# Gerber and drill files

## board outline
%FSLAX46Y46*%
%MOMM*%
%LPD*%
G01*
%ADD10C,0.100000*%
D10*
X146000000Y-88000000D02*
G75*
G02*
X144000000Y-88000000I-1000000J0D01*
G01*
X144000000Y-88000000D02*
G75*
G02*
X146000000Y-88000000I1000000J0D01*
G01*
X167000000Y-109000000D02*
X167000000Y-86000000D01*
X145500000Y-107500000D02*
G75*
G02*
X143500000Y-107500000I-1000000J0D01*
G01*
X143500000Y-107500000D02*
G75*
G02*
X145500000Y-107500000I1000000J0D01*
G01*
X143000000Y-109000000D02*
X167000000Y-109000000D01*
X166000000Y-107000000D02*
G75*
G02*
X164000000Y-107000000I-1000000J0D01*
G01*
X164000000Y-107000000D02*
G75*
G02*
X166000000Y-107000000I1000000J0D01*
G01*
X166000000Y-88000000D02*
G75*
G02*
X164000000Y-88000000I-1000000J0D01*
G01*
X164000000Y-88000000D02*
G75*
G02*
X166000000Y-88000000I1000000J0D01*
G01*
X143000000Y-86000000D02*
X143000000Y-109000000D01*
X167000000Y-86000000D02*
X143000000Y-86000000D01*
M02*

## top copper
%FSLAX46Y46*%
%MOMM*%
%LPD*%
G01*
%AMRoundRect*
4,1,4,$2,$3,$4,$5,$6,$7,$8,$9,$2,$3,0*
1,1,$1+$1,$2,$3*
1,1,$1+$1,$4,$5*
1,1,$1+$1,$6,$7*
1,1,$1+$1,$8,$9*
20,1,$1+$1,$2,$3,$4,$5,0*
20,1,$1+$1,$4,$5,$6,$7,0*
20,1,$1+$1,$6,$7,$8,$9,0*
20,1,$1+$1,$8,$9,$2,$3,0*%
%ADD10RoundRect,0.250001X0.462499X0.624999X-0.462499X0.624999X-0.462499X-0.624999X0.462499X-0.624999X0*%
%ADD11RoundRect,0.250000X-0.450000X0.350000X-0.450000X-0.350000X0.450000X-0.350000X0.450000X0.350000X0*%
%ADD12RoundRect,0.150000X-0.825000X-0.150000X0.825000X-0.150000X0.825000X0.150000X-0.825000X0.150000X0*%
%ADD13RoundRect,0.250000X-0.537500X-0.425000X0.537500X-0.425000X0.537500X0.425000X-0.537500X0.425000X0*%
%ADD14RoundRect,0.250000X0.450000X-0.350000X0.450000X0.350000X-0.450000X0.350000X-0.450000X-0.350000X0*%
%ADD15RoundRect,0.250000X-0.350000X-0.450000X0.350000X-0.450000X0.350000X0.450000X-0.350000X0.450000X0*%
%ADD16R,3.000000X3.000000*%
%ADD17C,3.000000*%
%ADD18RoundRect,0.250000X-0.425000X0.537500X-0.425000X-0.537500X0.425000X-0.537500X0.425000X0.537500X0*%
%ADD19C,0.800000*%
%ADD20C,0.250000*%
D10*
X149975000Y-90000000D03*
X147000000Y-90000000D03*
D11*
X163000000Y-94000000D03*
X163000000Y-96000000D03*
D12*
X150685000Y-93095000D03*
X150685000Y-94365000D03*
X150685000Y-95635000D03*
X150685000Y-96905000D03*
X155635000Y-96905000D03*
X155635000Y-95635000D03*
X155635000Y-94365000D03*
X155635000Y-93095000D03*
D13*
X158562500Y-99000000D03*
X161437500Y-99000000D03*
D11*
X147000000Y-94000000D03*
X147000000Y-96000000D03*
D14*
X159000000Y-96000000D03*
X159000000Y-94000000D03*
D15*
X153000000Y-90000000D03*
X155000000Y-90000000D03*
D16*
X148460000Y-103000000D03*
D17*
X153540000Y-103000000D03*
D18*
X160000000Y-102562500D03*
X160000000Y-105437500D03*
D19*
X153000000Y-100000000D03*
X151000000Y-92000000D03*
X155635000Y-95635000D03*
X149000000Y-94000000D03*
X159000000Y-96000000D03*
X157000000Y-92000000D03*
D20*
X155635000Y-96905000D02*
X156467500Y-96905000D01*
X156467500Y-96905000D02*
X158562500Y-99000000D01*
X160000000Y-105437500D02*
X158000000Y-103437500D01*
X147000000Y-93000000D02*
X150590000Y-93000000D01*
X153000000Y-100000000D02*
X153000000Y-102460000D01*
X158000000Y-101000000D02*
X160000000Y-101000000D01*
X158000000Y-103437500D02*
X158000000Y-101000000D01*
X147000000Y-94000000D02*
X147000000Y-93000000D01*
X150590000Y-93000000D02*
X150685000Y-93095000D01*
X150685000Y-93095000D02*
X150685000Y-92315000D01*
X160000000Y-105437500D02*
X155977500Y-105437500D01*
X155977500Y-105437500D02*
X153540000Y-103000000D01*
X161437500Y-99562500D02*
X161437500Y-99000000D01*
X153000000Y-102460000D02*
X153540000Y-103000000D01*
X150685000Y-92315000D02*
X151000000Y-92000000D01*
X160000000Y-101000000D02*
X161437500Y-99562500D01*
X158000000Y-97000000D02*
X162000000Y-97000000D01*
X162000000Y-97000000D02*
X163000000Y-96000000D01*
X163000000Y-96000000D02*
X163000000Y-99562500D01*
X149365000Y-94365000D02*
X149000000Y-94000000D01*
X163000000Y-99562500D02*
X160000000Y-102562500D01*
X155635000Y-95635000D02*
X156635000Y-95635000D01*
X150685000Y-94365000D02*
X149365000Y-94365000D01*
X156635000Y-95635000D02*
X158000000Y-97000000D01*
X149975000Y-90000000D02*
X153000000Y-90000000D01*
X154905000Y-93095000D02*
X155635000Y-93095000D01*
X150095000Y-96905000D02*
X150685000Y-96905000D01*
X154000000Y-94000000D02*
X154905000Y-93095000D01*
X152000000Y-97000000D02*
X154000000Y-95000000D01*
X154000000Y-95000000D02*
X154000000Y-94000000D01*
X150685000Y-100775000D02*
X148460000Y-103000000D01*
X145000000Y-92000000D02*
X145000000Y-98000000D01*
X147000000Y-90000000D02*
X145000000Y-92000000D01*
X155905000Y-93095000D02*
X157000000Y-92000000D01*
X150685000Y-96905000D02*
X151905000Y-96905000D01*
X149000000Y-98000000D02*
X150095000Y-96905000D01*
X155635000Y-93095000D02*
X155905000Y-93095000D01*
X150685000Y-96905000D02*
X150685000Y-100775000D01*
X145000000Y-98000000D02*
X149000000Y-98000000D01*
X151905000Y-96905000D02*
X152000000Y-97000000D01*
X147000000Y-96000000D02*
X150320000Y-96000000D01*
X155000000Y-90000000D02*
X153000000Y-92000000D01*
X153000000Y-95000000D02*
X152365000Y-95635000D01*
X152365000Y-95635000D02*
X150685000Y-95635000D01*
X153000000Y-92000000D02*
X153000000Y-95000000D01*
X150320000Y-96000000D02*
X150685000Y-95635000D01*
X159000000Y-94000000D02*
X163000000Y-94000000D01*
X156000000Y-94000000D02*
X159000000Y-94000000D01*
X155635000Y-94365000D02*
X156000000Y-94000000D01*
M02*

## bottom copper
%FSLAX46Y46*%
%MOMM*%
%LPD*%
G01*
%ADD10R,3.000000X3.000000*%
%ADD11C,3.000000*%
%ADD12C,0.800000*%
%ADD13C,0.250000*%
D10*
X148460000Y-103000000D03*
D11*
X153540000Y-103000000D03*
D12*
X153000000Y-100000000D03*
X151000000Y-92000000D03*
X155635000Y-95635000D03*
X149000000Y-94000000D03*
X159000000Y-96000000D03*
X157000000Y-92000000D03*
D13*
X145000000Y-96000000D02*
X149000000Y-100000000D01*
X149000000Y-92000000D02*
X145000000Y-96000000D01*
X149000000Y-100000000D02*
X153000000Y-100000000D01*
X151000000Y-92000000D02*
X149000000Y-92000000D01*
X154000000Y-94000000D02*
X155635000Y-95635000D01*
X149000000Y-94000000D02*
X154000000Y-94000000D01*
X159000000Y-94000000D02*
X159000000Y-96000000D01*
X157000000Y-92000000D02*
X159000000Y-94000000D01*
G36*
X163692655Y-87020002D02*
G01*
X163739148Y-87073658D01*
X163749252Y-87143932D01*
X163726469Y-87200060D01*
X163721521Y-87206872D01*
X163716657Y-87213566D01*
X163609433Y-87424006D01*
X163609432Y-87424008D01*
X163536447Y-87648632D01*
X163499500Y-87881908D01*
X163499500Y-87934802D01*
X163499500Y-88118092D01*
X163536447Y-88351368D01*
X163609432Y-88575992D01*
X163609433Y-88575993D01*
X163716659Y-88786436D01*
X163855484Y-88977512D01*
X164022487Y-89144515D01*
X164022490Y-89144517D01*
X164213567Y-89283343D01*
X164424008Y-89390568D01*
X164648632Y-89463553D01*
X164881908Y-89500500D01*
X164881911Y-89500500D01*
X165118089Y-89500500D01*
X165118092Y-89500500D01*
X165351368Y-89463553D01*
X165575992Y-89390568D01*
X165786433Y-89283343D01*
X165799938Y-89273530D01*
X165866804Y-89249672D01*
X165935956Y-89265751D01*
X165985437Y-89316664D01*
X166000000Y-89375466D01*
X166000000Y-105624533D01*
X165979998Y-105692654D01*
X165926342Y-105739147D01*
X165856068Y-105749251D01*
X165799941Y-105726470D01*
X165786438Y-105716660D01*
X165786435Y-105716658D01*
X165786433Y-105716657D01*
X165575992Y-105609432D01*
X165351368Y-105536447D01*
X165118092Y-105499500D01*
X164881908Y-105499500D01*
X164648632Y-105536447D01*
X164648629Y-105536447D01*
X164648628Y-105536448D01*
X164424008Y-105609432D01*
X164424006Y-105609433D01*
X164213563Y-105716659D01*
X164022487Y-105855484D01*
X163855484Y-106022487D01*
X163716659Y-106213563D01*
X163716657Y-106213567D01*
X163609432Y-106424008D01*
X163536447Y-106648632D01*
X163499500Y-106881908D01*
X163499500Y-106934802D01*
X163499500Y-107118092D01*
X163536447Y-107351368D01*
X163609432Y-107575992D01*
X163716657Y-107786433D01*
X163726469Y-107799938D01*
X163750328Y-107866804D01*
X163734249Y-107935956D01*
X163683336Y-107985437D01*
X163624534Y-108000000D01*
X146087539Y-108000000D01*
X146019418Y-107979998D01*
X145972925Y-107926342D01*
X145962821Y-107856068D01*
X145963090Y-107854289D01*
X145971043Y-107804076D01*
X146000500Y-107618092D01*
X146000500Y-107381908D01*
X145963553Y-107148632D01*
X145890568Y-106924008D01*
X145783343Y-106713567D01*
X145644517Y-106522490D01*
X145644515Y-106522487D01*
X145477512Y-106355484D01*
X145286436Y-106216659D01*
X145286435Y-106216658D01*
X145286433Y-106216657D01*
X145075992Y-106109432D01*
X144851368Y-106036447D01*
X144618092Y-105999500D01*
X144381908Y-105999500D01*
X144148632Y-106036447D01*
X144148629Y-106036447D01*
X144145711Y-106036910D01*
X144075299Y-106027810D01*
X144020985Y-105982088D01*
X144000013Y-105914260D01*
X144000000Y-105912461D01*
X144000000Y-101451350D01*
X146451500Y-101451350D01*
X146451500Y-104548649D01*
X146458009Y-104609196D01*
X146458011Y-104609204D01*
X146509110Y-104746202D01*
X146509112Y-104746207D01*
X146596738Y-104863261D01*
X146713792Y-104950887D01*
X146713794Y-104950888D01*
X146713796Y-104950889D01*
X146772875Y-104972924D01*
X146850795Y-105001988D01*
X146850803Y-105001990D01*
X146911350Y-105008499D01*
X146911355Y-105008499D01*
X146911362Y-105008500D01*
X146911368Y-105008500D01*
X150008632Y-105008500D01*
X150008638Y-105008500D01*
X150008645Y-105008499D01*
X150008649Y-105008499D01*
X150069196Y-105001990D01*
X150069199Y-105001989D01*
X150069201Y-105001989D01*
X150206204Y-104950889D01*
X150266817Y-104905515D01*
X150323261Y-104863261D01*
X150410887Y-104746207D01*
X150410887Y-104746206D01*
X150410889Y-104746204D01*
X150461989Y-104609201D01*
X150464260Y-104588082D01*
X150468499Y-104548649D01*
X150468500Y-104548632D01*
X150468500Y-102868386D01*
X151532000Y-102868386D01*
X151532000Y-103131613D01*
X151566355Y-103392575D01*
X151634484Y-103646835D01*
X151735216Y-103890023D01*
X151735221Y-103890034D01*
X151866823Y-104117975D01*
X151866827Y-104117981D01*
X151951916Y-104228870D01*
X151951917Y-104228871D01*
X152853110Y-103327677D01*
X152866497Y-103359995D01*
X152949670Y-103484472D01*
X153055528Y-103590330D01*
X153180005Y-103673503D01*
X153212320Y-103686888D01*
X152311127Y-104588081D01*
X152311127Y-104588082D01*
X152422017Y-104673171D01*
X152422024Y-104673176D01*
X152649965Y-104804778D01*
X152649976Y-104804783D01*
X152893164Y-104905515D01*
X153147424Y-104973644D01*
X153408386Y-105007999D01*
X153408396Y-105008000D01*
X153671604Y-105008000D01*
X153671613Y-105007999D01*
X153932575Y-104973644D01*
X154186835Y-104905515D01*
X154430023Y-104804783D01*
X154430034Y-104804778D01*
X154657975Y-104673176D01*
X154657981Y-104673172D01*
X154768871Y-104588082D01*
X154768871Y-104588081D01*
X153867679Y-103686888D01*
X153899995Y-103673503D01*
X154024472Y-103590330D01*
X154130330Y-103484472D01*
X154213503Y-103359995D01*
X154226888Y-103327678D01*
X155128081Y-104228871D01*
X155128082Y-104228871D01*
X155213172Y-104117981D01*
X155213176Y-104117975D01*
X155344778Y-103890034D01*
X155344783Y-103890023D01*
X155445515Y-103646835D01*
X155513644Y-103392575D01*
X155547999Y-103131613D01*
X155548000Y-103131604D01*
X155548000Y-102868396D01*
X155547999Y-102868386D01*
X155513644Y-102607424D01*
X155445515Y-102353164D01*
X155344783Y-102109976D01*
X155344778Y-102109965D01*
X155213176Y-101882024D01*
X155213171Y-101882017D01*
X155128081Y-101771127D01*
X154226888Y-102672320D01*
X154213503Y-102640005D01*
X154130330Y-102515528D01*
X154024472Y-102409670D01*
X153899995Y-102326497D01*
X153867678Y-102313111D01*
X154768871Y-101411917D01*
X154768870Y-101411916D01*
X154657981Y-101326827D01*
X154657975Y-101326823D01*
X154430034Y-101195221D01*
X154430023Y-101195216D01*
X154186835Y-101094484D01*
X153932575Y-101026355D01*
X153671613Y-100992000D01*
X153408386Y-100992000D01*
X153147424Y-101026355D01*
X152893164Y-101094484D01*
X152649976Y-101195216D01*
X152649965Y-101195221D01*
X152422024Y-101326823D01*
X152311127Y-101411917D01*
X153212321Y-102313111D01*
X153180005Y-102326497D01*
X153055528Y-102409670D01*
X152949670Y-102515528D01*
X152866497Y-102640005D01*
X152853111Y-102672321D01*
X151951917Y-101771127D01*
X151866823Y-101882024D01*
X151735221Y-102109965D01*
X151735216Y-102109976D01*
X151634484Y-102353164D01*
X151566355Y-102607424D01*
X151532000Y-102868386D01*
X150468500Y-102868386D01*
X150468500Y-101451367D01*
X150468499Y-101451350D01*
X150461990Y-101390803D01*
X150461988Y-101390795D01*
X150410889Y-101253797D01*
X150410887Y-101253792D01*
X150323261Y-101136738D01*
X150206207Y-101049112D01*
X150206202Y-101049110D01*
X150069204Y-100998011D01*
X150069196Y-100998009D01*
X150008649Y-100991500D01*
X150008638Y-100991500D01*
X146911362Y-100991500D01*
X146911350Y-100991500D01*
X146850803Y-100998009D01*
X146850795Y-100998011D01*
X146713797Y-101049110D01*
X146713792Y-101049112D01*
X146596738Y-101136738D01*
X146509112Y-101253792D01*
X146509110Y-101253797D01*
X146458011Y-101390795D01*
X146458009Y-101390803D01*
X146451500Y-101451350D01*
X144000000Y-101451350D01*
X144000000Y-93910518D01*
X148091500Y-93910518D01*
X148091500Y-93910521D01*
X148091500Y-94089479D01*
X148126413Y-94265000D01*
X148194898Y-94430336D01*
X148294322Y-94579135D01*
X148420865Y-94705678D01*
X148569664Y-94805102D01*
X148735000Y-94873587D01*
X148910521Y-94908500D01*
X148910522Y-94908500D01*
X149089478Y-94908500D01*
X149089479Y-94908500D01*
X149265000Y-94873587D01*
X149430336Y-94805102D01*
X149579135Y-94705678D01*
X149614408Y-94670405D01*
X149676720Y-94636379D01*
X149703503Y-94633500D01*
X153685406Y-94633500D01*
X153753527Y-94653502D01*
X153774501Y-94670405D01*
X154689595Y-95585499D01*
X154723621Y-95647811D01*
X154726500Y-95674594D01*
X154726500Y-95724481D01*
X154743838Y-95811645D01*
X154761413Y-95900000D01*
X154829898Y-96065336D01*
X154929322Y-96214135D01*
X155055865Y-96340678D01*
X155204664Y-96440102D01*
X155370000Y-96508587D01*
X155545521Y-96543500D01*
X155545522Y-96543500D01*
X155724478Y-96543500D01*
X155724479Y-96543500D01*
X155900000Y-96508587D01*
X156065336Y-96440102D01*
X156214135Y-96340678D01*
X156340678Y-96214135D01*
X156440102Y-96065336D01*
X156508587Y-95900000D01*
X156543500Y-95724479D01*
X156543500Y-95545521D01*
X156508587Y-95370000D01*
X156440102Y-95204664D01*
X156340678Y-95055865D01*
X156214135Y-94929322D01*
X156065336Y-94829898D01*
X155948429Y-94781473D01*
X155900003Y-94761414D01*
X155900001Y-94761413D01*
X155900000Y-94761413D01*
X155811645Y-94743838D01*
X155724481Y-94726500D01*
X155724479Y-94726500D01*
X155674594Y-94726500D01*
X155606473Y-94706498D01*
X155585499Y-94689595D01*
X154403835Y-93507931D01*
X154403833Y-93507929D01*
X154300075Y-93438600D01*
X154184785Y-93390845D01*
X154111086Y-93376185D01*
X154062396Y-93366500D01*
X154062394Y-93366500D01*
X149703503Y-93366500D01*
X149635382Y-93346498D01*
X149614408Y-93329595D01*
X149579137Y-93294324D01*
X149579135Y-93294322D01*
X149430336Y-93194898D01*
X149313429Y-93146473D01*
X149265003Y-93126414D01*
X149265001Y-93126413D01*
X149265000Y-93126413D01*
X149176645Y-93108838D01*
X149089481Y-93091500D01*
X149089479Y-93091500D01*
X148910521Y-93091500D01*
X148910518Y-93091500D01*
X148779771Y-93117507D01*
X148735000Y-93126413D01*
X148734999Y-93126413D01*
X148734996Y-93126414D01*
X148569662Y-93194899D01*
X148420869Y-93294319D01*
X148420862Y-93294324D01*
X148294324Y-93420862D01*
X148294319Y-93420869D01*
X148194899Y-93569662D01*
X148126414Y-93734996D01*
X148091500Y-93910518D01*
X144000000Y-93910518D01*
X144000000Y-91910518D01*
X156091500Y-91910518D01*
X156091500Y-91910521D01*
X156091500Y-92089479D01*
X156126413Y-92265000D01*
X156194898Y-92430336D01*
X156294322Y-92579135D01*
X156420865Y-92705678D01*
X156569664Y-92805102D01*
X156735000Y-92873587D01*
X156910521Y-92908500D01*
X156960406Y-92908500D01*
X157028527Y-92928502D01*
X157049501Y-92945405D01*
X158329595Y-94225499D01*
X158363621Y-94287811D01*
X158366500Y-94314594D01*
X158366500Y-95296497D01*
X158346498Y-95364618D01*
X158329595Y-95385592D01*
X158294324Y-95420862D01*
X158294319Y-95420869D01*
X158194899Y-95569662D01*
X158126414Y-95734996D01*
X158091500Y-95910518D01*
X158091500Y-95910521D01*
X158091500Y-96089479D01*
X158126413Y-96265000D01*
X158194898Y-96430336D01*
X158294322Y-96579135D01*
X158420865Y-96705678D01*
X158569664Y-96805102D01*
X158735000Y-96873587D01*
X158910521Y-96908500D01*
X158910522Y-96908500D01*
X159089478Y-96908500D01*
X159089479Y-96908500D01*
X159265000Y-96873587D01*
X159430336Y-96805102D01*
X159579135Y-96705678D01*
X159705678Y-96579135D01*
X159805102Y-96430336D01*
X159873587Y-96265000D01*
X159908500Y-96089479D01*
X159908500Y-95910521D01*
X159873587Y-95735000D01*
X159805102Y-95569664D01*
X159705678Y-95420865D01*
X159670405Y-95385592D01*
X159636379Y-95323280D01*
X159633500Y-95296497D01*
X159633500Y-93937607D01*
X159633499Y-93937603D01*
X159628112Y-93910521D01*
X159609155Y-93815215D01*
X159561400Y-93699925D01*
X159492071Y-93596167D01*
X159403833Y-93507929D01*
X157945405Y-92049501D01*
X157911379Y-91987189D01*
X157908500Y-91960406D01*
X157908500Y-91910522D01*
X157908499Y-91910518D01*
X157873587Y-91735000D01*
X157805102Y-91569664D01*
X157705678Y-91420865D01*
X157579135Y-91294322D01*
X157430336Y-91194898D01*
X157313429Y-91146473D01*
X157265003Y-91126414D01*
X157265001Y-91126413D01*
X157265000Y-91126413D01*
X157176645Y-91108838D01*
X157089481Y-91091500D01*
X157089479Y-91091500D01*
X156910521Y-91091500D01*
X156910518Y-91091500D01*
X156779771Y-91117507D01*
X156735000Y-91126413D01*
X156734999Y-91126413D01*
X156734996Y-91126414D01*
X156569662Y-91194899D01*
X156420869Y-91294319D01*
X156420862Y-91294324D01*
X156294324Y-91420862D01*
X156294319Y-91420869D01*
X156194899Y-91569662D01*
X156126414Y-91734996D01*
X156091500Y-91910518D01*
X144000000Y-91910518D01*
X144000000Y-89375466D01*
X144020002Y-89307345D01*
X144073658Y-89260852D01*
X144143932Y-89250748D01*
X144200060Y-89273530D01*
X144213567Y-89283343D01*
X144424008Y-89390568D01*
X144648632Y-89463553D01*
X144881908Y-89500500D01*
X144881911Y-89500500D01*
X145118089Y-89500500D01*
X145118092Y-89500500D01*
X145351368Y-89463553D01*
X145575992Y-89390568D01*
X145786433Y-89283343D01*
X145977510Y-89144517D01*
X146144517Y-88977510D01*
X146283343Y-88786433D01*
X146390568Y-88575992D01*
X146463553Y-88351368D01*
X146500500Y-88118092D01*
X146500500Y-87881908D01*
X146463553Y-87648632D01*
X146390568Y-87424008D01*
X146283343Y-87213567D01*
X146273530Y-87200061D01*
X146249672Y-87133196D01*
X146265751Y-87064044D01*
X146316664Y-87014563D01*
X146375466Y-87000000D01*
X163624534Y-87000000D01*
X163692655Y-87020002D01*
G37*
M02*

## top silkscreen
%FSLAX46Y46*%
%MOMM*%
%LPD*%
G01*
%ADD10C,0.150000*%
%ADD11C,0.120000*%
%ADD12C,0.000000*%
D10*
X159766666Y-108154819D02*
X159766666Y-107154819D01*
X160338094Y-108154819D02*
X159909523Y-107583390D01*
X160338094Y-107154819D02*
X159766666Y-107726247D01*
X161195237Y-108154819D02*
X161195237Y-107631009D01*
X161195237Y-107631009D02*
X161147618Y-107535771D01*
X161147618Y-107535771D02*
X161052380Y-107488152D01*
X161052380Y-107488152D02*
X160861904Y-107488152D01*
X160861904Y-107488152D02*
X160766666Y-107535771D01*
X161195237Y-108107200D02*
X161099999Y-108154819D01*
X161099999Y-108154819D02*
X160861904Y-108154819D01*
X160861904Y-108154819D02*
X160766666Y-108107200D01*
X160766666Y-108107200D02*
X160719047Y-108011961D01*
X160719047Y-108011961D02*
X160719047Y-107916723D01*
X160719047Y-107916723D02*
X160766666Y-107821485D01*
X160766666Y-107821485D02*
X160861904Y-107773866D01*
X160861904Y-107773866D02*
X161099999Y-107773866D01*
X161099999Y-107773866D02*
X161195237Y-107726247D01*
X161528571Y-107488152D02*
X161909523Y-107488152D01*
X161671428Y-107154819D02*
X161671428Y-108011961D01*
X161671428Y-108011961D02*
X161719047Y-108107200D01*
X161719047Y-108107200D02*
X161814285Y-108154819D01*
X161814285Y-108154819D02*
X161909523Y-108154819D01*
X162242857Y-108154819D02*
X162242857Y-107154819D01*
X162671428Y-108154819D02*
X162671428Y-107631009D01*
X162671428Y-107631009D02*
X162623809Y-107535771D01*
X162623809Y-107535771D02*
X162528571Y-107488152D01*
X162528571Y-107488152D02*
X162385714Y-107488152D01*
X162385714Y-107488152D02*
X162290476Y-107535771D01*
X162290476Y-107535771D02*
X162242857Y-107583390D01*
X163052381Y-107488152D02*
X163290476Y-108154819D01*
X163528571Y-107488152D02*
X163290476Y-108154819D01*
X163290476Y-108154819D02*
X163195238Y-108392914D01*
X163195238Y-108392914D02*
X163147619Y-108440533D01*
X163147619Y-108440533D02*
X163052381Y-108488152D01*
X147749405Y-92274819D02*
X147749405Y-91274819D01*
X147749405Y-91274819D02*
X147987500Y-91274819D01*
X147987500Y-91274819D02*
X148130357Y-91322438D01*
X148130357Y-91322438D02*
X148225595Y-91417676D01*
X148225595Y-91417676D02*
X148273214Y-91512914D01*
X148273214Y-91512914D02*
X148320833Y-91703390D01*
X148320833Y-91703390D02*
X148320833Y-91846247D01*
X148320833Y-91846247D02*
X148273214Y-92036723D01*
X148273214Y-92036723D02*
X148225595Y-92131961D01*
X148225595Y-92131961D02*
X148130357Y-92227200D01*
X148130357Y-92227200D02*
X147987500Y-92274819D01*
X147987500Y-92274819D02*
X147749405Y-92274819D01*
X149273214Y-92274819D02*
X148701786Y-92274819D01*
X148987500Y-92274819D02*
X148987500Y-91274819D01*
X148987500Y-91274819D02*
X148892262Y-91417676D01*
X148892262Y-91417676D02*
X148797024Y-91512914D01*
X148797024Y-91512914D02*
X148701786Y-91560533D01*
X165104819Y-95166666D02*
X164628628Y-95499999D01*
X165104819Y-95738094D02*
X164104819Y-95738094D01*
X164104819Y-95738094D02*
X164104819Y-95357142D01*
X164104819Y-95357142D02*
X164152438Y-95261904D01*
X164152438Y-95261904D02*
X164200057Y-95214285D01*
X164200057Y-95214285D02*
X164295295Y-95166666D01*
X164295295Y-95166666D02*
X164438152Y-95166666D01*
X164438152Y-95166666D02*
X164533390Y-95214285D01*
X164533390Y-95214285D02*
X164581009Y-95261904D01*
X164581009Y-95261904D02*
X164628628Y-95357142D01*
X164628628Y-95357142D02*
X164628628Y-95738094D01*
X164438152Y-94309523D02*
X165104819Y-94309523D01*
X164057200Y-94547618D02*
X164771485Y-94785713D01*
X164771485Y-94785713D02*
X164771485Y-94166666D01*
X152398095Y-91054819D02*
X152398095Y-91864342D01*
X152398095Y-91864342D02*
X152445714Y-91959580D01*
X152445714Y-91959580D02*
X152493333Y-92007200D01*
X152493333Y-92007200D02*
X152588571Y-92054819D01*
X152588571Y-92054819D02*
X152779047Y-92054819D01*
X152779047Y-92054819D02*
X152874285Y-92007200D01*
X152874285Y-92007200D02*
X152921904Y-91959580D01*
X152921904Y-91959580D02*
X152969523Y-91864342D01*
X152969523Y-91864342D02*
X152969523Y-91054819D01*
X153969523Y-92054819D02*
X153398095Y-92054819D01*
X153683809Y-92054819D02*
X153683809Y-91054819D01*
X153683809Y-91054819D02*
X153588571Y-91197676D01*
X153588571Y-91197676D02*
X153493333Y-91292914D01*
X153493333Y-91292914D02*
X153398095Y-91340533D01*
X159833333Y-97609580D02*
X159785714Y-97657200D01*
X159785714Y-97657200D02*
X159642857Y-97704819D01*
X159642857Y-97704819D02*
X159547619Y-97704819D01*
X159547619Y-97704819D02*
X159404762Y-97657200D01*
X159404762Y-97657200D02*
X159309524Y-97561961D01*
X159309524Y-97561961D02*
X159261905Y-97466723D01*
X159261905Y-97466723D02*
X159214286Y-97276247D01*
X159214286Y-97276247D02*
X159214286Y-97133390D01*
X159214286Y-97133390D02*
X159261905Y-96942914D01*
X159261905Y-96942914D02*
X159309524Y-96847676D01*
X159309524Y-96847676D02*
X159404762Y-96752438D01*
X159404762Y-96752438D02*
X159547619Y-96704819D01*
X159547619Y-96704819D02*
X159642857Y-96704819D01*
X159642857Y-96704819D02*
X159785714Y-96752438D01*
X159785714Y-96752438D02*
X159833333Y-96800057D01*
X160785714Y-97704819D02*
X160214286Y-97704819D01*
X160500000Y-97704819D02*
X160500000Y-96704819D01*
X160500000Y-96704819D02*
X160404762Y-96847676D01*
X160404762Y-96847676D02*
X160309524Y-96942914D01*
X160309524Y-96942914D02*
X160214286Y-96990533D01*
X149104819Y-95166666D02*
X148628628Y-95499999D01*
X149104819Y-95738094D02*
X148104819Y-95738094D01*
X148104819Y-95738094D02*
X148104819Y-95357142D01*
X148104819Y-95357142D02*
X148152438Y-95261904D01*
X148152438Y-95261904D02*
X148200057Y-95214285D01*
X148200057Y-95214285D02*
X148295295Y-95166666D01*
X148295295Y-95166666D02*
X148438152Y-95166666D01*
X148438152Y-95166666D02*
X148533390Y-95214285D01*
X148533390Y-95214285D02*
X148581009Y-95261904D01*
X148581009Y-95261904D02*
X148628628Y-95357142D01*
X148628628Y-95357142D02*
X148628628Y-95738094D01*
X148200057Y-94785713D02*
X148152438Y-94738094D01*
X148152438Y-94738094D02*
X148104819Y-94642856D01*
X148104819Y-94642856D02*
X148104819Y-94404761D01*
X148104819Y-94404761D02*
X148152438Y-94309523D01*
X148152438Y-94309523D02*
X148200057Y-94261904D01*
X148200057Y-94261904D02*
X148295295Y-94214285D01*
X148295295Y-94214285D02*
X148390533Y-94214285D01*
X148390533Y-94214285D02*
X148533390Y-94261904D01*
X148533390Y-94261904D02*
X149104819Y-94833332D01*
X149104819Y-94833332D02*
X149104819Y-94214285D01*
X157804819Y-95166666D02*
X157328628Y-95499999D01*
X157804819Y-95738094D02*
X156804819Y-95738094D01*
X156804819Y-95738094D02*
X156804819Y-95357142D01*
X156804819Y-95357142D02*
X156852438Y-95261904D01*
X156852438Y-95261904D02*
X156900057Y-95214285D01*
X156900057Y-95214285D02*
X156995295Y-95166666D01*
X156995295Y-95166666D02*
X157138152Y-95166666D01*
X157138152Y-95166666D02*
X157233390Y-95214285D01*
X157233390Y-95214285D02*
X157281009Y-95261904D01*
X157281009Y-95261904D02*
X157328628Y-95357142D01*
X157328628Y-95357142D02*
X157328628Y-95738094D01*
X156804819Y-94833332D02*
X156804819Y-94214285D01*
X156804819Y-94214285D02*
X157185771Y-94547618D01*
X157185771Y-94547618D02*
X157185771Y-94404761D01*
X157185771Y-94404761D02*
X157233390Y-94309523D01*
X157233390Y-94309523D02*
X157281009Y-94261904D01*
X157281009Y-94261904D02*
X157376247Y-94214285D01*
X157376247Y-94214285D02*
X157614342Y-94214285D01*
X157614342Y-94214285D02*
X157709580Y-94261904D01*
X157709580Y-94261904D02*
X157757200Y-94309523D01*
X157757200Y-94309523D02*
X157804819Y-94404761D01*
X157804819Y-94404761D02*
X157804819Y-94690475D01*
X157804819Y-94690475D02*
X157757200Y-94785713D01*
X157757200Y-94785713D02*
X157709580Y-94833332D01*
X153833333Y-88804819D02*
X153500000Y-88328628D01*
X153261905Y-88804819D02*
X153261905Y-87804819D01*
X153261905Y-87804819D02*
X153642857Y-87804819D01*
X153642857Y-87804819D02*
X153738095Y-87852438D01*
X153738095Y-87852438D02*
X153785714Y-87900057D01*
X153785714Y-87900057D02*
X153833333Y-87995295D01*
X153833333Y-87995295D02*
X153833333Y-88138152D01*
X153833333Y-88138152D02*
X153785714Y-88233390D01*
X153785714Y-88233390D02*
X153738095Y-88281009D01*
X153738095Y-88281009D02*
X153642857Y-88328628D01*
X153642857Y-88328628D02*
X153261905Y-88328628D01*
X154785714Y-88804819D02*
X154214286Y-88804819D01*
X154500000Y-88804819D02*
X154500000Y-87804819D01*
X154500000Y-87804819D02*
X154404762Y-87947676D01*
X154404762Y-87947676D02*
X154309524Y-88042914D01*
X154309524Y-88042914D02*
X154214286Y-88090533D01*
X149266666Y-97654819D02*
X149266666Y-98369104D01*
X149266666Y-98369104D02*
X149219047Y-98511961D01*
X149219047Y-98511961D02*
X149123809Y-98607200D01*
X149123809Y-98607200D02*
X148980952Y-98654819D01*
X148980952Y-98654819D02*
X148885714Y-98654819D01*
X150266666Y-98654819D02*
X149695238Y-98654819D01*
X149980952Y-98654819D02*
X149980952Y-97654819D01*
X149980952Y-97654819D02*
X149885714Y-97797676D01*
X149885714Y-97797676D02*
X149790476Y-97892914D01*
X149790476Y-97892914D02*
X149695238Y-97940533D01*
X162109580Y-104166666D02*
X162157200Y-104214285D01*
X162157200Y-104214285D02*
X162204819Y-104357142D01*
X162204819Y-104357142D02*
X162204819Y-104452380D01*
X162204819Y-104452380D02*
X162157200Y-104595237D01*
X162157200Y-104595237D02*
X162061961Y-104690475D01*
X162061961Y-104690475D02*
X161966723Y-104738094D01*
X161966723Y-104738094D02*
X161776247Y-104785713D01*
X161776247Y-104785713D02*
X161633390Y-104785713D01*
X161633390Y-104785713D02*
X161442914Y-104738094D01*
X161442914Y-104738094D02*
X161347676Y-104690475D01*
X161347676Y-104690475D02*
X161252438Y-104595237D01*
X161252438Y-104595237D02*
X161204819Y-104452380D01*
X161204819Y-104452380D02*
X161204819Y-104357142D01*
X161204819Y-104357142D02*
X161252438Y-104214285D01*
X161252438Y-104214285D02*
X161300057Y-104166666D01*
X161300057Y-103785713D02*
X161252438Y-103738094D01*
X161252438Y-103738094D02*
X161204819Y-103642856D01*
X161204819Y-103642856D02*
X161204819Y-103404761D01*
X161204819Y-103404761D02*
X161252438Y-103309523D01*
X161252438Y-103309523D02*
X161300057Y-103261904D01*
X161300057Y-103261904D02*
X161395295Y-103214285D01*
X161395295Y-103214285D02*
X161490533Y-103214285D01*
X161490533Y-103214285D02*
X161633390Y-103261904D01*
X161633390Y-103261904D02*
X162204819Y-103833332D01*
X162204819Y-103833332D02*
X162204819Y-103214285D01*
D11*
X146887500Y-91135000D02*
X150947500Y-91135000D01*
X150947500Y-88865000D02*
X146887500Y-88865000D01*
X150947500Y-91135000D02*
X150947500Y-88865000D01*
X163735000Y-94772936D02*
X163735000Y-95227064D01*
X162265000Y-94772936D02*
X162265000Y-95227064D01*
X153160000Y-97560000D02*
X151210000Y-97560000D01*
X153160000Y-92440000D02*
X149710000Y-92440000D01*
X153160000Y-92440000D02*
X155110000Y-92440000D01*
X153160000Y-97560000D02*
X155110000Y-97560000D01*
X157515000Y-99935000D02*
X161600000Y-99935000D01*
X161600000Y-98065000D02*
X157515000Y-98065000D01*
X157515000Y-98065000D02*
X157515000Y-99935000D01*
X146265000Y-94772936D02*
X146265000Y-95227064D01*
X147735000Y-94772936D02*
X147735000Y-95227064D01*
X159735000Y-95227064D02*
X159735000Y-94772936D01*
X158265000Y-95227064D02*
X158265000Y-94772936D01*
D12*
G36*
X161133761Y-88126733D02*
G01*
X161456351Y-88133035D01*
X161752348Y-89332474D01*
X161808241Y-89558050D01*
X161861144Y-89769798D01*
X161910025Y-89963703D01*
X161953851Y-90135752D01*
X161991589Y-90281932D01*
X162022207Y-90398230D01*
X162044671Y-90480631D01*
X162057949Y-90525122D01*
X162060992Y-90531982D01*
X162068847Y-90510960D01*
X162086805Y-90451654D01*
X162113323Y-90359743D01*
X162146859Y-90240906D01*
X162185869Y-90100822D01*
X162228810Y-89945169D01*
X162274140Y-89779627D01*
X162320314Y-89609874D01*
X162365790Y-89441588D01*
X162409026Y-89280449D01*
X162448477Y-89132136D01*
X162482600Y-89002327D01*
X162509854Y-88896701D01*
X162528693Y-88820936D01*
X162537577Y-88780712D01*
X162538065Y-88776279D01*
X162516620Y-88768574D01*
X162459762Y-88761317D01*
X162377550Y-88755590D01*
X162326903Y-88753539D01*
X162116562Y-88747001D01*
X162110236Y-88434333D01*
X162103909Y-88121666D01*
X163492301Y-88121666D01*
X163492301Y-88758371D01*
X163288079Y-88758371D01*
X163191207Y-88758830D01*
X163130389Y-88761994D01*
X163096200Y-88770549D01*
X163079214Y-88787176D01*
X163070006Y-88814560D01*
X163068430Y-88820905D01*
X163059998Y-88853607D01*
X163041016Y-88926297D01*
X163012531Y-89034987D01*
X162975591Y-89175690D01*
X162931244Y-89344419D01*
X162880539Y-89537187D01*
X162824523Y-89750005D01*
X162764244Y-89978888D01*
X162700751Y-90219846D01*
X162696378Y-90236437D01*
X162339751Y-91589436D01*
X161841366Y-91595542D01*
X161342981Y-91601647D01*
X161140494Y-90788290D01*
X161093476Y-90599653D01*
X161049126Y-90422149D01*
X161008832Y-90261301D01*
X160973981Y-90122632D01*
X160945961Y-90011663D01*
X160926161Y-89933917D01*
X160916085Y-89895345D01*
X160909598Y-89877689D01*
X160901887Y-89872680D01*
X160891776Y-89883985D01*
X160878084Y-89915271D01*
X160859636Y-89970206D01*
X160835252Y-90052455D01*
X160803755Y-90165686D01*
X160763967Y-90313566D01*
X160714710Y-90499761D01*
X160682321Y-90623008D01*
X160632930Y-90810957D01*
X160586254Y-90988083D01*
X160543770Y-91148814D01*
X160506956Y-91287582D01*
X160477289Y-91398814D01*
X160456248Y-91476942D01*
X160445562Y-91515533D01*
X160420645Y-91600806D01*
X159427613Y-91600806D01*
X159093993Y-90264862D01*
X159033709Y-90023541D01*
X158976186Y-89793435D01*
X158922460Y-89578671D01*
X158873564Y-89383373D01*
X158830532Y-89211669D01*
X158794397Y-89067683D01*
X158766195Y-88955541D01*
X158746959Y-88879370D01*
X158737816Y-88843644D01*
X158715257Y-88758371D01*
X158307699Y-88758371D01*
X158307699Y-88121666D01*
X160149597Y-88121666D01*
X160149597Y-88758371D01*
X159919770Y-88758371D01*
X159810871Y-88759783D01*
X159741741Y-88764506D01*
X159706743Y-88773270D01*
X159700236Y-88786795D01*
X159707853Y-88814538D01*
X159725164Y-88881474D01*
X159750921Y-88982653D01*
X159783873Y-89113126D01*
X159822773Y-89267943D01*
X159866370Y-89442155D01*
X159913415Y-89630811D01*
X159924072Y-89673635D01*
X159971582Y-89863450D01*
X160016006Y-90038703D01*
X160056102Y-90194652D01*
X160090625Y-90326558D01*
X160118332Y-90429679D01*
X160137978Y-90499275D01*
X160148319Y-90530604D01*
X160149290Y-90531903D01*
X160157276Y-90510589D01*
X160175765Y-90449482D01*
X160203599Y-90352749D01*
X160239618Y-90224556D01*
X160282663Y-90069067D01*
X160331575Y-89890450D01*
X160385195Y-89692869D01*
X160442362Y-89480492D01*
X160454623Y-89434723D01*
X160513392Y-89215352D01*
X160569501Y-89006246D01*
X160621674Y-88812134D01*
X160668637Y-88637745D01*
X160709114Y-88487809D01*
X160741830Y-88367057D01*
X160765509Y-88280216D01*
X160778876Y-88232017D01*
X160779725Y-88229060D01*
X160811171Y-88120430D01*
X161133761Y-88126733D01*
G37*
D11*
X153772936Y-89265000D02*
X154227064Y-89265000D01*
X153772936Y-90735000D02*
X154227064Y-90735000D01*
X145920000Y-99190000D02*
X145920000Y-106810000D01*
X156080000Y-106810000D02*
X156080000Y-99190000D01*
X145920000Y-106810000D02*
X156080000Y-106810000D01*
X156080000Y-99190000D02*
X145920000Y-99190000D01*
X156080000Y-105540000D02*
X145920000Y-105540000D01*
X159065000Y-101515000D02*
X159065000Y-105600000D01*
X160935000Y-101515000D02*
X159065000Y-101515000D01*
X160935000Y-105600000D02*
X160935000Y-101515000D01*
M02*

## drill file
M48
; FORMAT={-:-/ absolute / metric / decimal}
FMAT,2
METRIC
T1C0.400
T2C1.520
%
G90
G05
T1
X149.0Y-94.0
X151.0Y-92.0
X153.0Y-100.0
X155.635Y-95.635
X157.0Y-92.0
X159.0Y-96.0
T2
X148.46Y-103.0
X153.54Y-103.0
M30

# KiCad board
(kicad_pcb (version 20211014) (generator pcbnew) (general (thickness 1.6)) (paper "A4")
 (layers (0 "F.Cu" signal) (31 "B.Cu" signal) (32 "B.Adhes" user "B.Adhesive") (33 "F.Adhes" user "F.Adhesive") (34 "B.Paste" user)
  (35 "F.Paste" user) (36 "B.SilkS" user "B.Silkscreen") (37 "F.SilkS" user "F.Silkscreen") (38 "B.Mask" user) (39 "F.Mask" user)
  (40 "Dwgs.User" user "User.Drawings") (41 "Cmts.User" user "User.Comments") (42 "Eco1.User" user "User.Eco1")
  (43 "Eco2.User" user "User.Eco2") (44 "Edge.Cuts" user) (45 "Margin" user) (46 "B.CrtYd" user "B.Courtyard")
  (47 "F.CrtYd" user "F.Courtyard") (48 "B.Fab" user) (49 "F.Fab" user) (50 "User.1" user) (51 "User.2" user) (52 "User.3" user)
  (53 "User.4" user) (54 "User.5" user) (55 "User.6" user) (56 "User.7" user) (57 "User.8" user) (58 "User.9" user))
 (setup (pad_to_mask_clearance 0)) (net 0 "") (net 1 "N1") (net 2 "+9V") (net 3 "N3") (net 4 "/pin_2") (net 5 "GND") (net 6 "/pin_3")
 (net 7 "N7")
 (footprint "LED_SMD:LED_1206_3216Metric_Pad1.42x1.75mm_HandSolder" (layer "F.Cu") (at 148.4875 90 180)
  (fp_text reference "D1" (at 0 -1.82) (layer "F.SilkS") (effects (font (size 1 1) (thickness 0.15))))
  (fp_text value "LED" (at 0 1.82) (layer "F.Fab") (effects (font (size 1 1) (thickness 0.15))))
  (fp_line (start 1.6 -1.135) (end -2.46 -1.135) (layer "F.SilkS") (width 0.12))
  (fp_line (start -2.46 1.135) (end 1.6 1.135) (layer "F.SilkS") (width 0.12))
  (fp_line (start -2.46 -1.135) (end -2.46 1.135) (layer "F.SilkS") (width 0.12))
  (pad "1" smd roundrect (at -1.4875 0 180) (size 1.425 1.75) (layers "F.Cu" "F.Paste" "F.Mask") (roundrect_rratio 0.175439) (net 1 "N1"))
  (pad "2" smd roundrect (at 1.4875 0 180) (size 1.425 1.75) (layers "F.Cu" "F.Paste" "F.Mask") (roundrect_rratio 0.175439) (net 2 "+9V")))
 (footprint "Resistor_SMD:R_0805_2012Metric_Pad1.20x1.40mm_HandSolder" (layer "F.Cu") (at 163 95 -90)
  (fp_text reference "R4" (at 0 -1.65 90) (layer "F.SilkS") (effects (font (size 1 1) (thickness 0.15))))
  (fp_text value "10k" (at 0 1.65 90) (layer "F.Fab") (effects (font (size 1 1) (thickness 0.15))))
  (fp_line (start -0.227064 -0.735) (end 0.227064 -0.735) (layer "F.SilkS") (width 0.12))
  (fp_line (start -0.227064 0.735) (end 0.227064 0.735) (layer "F.SilkS") (width 0.12))
  (pad "1" smd roundrect (at -1 0 270) (size 1.2 1.4) (layers "F.Cu" "F.Paste" "F.Mask") (roundrect_rratio 0.208333) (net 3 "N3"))
  (pad "2" smd roundrect (at 1 0 270) (size 1.2 1.4) (layers "F.Cu" "F.Paste" "F.Mask") (roundrect_rratio 0.208333) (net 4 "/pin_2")))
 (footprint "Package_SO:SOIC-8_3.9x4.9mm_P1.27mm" (layer "F.Cu") (at 153.16 95)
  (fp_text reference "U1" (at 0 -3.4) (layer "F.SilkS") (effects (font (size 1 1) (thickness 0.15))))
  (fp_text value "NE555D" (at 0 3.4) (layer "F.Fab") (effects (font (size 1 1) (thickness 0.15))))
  (fp_line (start 0 2.56) (end -1.95 2.56) (layer "F.SilkS") (width 0.12))
  (fp_line (start 0 -2.56) (end -3.45 -2.56) (layer "F.SilkS") (width 0.12))
  (fp_line (start 0 -2.56) (end 1.95 -2.56) (layer "F.SilkS") (width 0.12))
  (fp_line (start 0 2.56) (end 1.95 2.56) (layer "F.SilkS") (width 0.12))
  (pad "1" smd roundrect (at -2.475 -1.905) (size 1.95 0.6) (layers "F.Cu" "F.Paste" "F.Mask") (roundrect_rratio 0.25) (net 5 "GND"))
  (pad "2" smd roundrect (at -2.475 -0.635) (size 1.95 0.6) (layers "F.Cu" "F.Paste" "F.Mask") (roundrect_rratio 0.25) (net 4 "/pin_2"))
  (pad "3" smd roundrect (at -2.475 0.635) (size 1.95 0.6) (layers "F.Cu" "F.Paste" "F.Mask") (roundrect_rratio 0.25) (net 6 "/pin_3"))
  (pad "4" smd roundrect (at -2.475 1.905) (size 1.95 0.6) (layers "F.Cu" "F.Paste" "F.Mask") (roundrect_rratio 0.25) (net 2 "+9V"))
  (pad "5" smd roundrect (at 2.475 1.905) (size 1.95 0.6) (layers "F.Cu" "F.Paste" "F.Mask") (roundrect_rratio 0.25) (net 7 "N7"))
  (pad "6" smd roundrect (at 2.475 0.635) (size 1.95 0.6) (layers "F.Cu" "F.Paste" "F.Mask") (roundrect_rratio 0.25) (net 4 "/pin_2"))
  (pad "7" smd roundrect (at 2.475 -0.635) (size 1.95 0.6) (layers "F.Cu" "F.Paste" "F.Mask") (roundrect_rratio 0.25) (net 3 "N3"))
  (pad "8" smd roundrect (at 2.475 -1.905) (size 1.95 0.6) (layers "F.Cu" "F.Paste" "F.Mask") (roundrect_rratio 0.25) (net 2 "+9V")))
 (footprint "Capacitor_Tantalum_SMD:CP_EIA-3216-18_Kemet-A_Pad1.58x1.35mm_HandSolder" (layer "F.Cu") (at 160 99)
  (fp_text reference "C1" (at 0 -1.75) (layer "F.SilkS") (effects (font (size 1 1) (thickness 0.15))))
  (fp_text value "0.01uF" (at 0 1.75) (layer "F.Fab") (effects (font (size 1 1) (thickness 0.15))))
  (fp_line (start -2.485 0.935) (end 1.6 0.935) (layer "F.SilkS") (width 0.12))
  (fp_line (start 1.6 -0.935) (end -2.485 -0.935) (layer "F.SilkS") (width 0.12))
  (fp_line (start -2.485 -0.935) (end -2.485 0.935) (layer "F.SilkS") (width 0.12))
  (pad "1" smd roundrect (at -1.4375 0) (size 1.575 1.35) (layers "F.Cu" "F.Paste" "F.Mask") (roundrect_rratio 0.185185) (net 7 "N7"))
  (pad "2" smd roundrect (at 1.4375 0) (size 1.575 1.35) (layers "F.Cu" "F.Paste" "F.Mask") (roundrect_rratio 0.185185) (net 5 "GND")))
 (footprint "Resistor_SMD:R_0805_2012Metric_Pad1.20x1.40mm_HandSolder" (layer "F.Cu") (at 147 95 -90)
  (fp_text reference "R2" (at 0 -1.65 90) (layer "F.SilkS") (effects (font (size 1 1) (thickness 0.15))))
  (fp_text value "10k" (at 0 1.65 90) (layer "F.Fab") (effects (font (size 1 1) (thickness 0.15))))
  (fp_line (start -0.227064 0.735) (end 0.227064 0.735) (layer "F.SilkS") (width 0.12))
  (fp_line (start -0.227064 -0.735) (end 0.227064 -0.735) (layer "F.SilkS") (width 0.12))
  (pad "1" smd roundrect (at -1 0 270) (size 1.2 1.4) (layers "F.Cu" "F.Paste" "F.Mask") (roundrect_rratio 0.208333) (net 5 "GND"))
  (pad "2" smd roundrect (at 1 0 270) (size 1.2 1.4) (layers "F.Cu" "F.Paste" "F.Mask") (roundrect_rratio 0.208333) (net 6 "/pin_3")))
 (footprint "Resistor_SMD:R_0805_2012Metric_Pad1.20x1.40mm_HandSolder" (layer "F.Cu") (at 159 95 90)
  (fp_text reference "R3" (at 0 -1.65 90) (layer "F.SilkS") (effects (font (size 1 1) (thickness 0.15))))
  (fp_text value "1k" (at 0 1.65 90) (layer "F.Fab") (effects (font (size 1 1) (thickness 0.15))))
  (fp_line (start -0.227064 0.735) (end 0.227064 0.735) (layer "F.SilkS") (width 0.12))
  (fp_line (start -0.227064 -0.735) (end 0.227064 -0.735) (layer "F.SilkS") (width 0.12))
  (pad "1" smd roundrect (at -1 0 90) (size 1.2 1.4) (layers "F.Cu" "F.Paste" "F.Mask") (roundrect_rratio 0.208333) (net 2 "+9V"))
  (pad "2" smd roundrect (at 1 0 90) (size 1.2 1.4) (layers "F.Cu" "F.Paste" "F.Mask") (roundrect_rratio 0.208333) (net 3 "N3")))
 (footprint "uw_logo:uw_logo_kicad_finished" (layer "F.Cu") (at 160.9 90.1)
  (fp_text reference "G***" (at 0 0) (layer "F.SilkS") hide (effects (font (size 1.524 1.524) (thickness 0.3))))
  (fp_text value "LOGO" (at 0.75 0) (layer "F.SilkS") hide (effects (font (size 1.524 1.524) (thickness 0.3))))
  (fp_poly
   (pts (xy 0.233761 -1.973267) (xy 0.556351 -1.966965) (xy 0.852348 -0.767526) (xy 0.908241 -0.54195) (xy 0.961144 -0.330202)
    (xy 1.010025 -0.136297) (xy 1.053851 0.035752) (xy 1.091589 0.181932) (xy 1.122207 0.29823) (xy 1.144671 0.380631)
    (xy 1.157949 0.425122) (xy 1.160992 0.431982) (xy 1.168847 0.41096) (xy 1.186805 0.351654) (xy 1.213323 0.259743) (xy 1.246859 0.140906)
    (xy 1.285869 0.000822) (xy 1.32881 -0.154831) (xy 1.37414 -0.320373) (xy 1.420314 -0.490126) (xy 1.46579 -0.658412)
    (xy 1.509026 -0.819551) (xy 1.548477 -0.967864) (xy 1.5826 -1.097673) (xy 1.609854 -1.203299) (xy 1.628693 -1.279064)
    (xy 1.637577 -1.319288) (xy 1.638065 -1.323721) (xy 1.61662 -1.331426) (xy 1.559762 -1.338683) (xy 1.47755 -1.34441)
    (xy 1.426903 -1.346461) (xy 1.216562 -1.352999) (xy 1.210236 -1.665667) (xy 1.203909 -1.978334) (xy 2.592301 -1.978334)
    (xy 2.592301 -1.341629) (xy 2.388079 -1.341629) (xy 2.291207 -1.34117) (xy 2.230389 -1.338006) (xy 2.1962 -1.329451)
    (xy 2.179214 -1.312824) (xy 2.170006 -1.28544) (xy 2.16843 -1.279095) (xy 2.159998 -1.246393) (xy 2.141016 -1.173703)
    (xy 2.112531 -1.065013) (xy 2.075591 -0.92431) (xy 2.031244 -0.755581) (xy 1.980539 -0.562813) (xy 1.924523 -0.349995)
    (xy 1.864244 -0.121112) (xy 1.800751 0.119846) (xy 1.796378 0.136437) (xy 1.439751 1.489436) (xy 0.941366 1.495542)
    (xy 0.442981 1.501647) (xy 0.240494 0.68829) (xy 0.193476 0.499653) (xy 0.149126 0.322149) (xy 0.108832 0.161301) (xy 0.073981 0.022632)
    (xy 0.045961 -0.088337) (xy 0.026161 -0.166083) (xy 0.016085 -0.204655) (xy 0.009598 -0.222311) (xy 0.001887 -0.22732)
    (xy -0.008224 -0.216015) (xy -0.021916 -0.184729) (xy -0.040364 -0.129794) (xy -0.064748 -0.047545) (xy -0.096245 0.065686)
    (xy -0.136033 0.213566) (xy -0.18529 0.399761) (xy -0.217679 0.523008) (xy -0.26707 0.710957) (xy -0.313746 0.888083)
    (xy -0.35623 1.048814) (xy -0.393044 1.187582) (xy -0.422711 1.298814) (xy -0.443752 1.376942) (xy -0.454438 1.415533)
    (xy -0.479355 1.500806) (xy -1.472387 1.500806) (xy -1.806007 0.164862) (xy -1.866291 -0.076459) (xy -1.923814 -0.306565)
    (xy -1.97754 -0.521329) (xy -2.026436 -0.716627) (xy -2.069468 -0.888331) (xy -2.105603 -1.032317) (xy -2.133805 -1.144459)
    (xy -2.153041 -1.22063) (xy -2.162184 -1.256356) (xy -2.184743 -1.341629) (xy -2.592301 -1.341629) (xy -2.592301 -1.978334)
    (xy -0.750403 -1.978334) (xy -0.750403 -1.341629) (xy -0.98023 -1.341629) (xy -1.089129 -1.340217) (xy -1.158259 -1.335494)
    (xy -1.193257 -1.32673) (xy -1.199764 -1.313205) (xy -1.192147 -1.285462) (xy -1.174836 -1.218526) (xy -1.149079 -1.117347)
    (xy -1.116127 -0.986874) (xy -1.077227 -0.832057) (xy -1.03363 -0.657845) (xy -0.986585 -0.469189) (xy -0.975928 -0.426365)
    (xy -0.928418 -0.23655) (xy -0.883994 -0.061297) (xy -0.843898 0.094652) (xy -0.809375 0.226558) (xy -0.781668 0.329679)
    (xy -0.762022 0.399275) (xy -0.751681 0.430604) (xy -0.75071 0.431903) (xy -0.742724 0.410589) (xy -0.724235 0.349482)
    (xy -0.696401 0.252749) (xy -0.660382 0.124556) (xy -0.617337 -0.030933) (xy -0.568425 -0.20955) (xy -0.514805 -0.407131)
    (xy -0.457638 -0.619508) (xy -0.445377 -0.665277) (xy -0.386608 -0.884648) (xy -0.330499 -1.093754) (xy -0.278326 -1.287866)
    (xy -0.231363 -1.462255) (xy -0.190886 -1.612191) (xy -0.15817 -1.732943) (xy -0.134491 -1.819784) (xy -0.121124 -1.867983)
    (xy -0.120275 -1.87094) (xy -0.088829 -1.97957))
   (layer "F.SilkS") (width 0) (fill solid)))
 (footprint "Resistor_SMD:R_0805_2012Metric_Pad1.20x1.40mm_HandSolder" (layer "F.Cu") (at 154 90)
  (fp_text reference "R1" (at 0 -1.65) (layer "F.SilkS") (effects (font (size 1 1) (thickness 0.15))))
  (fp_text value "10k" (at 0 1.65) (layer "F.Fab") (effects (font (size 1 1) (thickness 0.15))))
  (fp_line (start -0.227064 -0.735) (end 0.227064 -0.735) (layer "F.SilkS") (width 0.12))
  (fp_line (start -0.227064 0.735) (end 0.227064 0.735) (layer "F.SilkS") (width 0.12))
  (pad "1" smd roundrect (at -1 0) (size 1.2 1.4) (layers "F.Cu" "F.Paste" "F.Mask") (roundrect_rratio 0.208333) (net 1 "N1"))
  (pad "2" smd roundrect (at 1 0) (size 1.2 1.4) (layers "F.Cu" "F.Paste" "F.Mask") (roundrect_rratio 0.208333) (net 6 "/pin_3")))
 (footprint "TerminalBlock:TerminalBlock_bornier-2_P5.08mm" (layer "F.Cu") (at 148.46 103)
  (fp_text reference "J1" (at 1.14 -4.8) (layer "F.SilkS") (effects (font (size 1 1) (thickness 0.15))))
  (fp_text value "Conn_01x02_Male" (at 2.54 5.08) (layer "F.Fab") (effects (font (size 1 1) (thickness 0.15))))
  (fp_line (start -2.54 -3.81) (end -2.54 3.81) (layer "F.SilkS") (width 0.12))
  (fp_line (start 7.62 3.81) (end 7.62 -3.81) (layer "F.SilkS") (width 0.12))
  (fp_line (start -2.54 3.81) (end 7.62 3.81) (layer "F.SilkS") (width 0.12))
  (fp_line (start 7.62 -3.81) (end -2.54 -3.81) (layer "F.SilkS") (width 0.12))
  (fp_line (start 7.62 2.54) (end -2.54 2.54) (layer "F.SilkS") (width 0.12))
  (pad "1" thru_hole rect (at 0 0) (size 3 3) (drill 1.52) (layers *.Cu *.Mask) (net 2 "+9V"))
  (pad "2" thru_hole circle (at 5.08 0) (size 3 3) (drill 1.52) (layers *.Cu *.Mask) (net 5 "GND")))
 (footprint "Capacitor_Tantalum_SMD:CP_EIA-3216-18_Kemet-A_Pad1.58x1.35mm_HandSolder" (layer "F.Cu") (at 160 104 -90)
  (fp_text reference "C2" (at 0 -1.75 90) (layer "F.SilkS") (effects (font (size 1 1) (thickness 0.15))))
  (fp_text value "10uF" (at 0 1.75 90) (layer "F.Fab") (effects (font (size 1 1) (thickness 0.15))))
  (fp_line (start -2.485 0.935) (end 1.6 0.935) (layer "F.SilkS") (width 0.12))
  (fp_line (start -2.485 -0.935) (end -2.485 0.935) (layer "F.SilkS") (width 0.12))
  (fp_line (start 1.6 -0.935) (end -2.485 -0.935) (layer "F.SilkS") (width 0.12))
  (pad "1" smd roundrect (at -1.4375 0 270) (size 1.575 1.35) (layers "F.Cu" "F.Paste" "F.Mask") (roundrect_rratio 0.185185)
   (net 4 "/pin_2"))
  (pad "2" smd roundrect (at 1.4375 0 270) (size 1.575 1.35) (layers "F.Cu" "F.Paste" "F.Mask") (roundrect_rratio 0.185185) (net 5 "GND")))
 (gr_circle (center 145 88) (end 144 88) (layer "Edge.Cuts") (width 0.1) (fill none))
 (gr_line (start 167 109) (end 167 86) (layer "Edge.Cuts") (width 0.1))
 (gr_circle (center 144.5 107.5) (end 145.5 107.5) (layer "Edge.Cuts") (width 0.1) (fill none))
 (gr_line (start 143 109) (end 167 109) (layer "Edge.Cuts") (width 0.1))
 (gr_circle (center 165 107) (end 166 107) (layer "Edge.Cuts") (width 0.1) (fill none))
 (gr_circle (center 165 88) (end 165 89) (layer "Edge.Cuts") (width 0.1) (fill none))
 (gr_line (start 143 86) (end 143 109) (layer "Edge.Cuts") (width 0.1))
 (gr_line (start 167 86) (end 143 86) (layer "Edge.Cuts") (width 0.1))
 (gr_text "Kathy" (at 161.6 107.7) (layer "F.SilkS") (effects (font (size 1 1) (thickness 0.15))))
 (segment (start 155.635 96.905) (end 156.4675 96.905) (width 0.25) (layer "F.Cu") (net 7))
 (segment (start 156.4675 96.905) (end 158.5625 99) (width 0.25) (layer "F.Cu") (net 7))
 (segment (start 160 105.4375) (end 158 103.4375) (width 0.25) (layer "F.Cu") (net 5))
 (segment (start 147 93) (end 150.59 93) (width 0.25) (layer "F.Cu") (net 5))
 (segment (start 153 100) (end 153 102.46) (width 0.25) (layer "F.Cu") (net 5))
 (segment (start 158 101) (end 160 101) (width 0.25) (layer "F.Cu") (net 5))
 (segment (start 158 103.4375) (end 158 101) (width 0.25) (layer "F.Cu") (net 5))
 (segment (start 147 94) (end 147 93) (width 0.25) (layer "F.Cu") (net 5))
 (segment (start 150.59 93) (end 150.685 93.095) (width 0.25) (layer "F.Cu") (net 5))
 (segment (start 150.685 93.095) (end 150.685 92.315) (width 0.25) (layer "F.Cu") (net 5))
 (segment (start 160 105.4375) (end 155.9775 105.4375) (width 0.25) (layer "F.Cu") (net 5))
 (segment (start 155.9775 105.4375) (end 153.54 103) (width 0.25) (layer "F.Cu") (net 5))
 (segment (start 161.4375 99.5625) (end 161.4375 99) (width 0.25) (layer "F.Cu") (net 5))
 (segment (start 153 102.46) (end 153.54 103) (width 0.25) (layer "F.Cu") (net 5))
 (segment (start 150.685 92.315) (end 151 92) (width 0.25) (layer "F.Cu") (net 5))
 (segment (start 160 101) (end 161.4375 99.5625) (width 0.25) (layer "F.Cu") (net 5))
 (via (at 153 100) (size 0.8) (drill 0.4) (layers "F.Cu" "B.Cu") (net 5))
 (via (at 151 92) (size 0.8) (drill 0.4) (layers "F.Cu" "B.Cu") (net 5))
 (segment (start 145 96) (end 149 100) (width 0.25) (layer "B.Cu") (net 5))
 (segment (start 149 92) (end 145 96) (width 0.25) (layer "B.Cu") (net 5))
 (segment (start 149 100) (end 153 100) (width 0.25) (layer "B.Cu") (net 5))
 (segment (start 151 92) (end 149 92) (width 0.25) (layer "B.Cu") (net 5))
 (segment (start 158 97) (end 162 97) (width 0.25) (layer "F.Cu") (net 4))
 (segment (start 162 97) (end 163 96) (width 0.25) (layer "F.Cu") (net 4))
 (segment (start 163 96) (end 163 99.5625) (width 0.25) (layer "F.Cu") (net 4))
 (segment (start 149.365 94.365) (end 149 94) (width 0.25) (layer "F.Cu") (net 4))
 (segment (start 163 99.5625) (end 160 102.5625) (width 0.25) (layer "F.Cu") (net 4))
 (segment (start 155.635 95.635) (end 156.635 95.635) (width 0.25) (layer "F.Cu") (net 4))
 (segment (start 150.685 94.365) (end 149.365 94.365) (width 0.25) (layer "F.Cu") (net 4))
 (segment (start 156.635 95.635) (end 158 97) (width 0.25) (layer "F.Cu") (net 4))
 (via (at 155.635 95.635) (size 0.8) (drill 0.4) (layers "F.Cu" "B.Cu") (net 4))
 (via (at 149 94) (size 0.8) (drill 0.4) (layers "F.Cu" "B.Cu") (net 4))
 (segment (start 154 94) (end 155.635 95.635) (width 0.25) (layer "B.Cu") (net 4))
 (segment (start 149 94) (end 154 94) (width 0.25) (layer "B.Cu") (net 4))
 (segment (start 149.975 90) (end 153 90) (width 0.25) (layer "F.Cu") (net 1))
 (segment (start 154.905 93.095) (end 155.635 93.095) (width 0.25) (layer "F.Cu") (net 2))
 (segment (start 150.095 96.905) (end 150.685 96.905) (width 0.25) (layer "F.Cu") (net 2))
 (segment (start 154 94) (end 154.905 93.095) (width 0.25) (layer "F.Cu") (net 2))
 (segment (start 152 97) (end 154 95) (width 0.25) (layer "F.Cu") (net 2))
 (segment (start 154 95) (end 154 94) (width 0.25) (layer "F.Cu") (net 2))
 (segment (start 150.685 100.775) (end 148.46 103) (width 0.25) (layer "F.Cu") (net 2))
 (segment (start 145 92) (end 145 98) (width 0.25) (layer "F.Cu") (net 2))
 (segment (start 147 90) (end 145 92) (width 0.25) (layer "F.Cu") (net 2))
 (segment (start 155.905 93.095) (end 157 92) (width 0.25) (layer "F.Cu") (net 2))
 (segment (start 150.685 96.905) (end 151.905 96.905) (width 0.25) (layer "F.Cu") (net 2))
 (segment (start 149 98) (end 150.095 96.905) (width 0.25) (layer "F.Cu") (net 2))
 (segment (start 155.635 93.095) (end 155.905 93.095) (width 0.25) (layer "F.Cu") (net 2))
 (segment (start 150.685 96.905) (end 150.685 100.775) (width 0.25) (layer "F.Cu") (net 2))
 (segment (start 145 98) (end 149 98) (width 0.25) (layer "F.Cu") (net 2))
 (segment (start 151.905 96.905) (end 152 97) (width 0.25) (layer "F.Cu") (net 2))
 (via (at 159 96) (size 0.8) (drill 0.4) (layers "F.Cu" "B.Cu") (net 2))
 (via (at 157 92) (size 0.8) (drill 0.4) (layers "F.Cu" "B.Cu") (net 2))
 (segment (start 159 94) (end 159 96) (width 0.25) (layer "B.Cu") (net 2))
 (segment (start 157 92) (end 159 94) (width 0.25) (layer "B.Cu") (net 2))
 (segment (start 147 96) (end 150.32 96) (width 0.25) (layer "F.Cu") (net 6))
 (segment (start 155 90) (end 153 92) (width 0.25) (layer "F.Cu") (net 6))
 (segment (start 153 95) (end 152.365 95.635) (width 0.25) (layer "F.Cu") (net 6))
 (segment (start 152.365 95.635) (end 150.685 95.635) (width 0.25) (layer "F.Cu") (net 6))
 (segment (start 153 92) (end 153 95) (width 0.25) (layer "F.Cu") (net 6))
 (segment (start 150.32 96) (end 150.685 95.635) (width 0.25) (layer "F.Cu") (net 6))
 (segment (start 159 94) (end 163 94) (width 0.25) (layer "F.Cu") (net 3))
 (segment (start 156 94) (end 159 94) (width 0.25) (layer "F.Cu") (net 3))
 (segment (start 155.635 94.365) (end 156 94) (width 0.25) (layer "F.Cu") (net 3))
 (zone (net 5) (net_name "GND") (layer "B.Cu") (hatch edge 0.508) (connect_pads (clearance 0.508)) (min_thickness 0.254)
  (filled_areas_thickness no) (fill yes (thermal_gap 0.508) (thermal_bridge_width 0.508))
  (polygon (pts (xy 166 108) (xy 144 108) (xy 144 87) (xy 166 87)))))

